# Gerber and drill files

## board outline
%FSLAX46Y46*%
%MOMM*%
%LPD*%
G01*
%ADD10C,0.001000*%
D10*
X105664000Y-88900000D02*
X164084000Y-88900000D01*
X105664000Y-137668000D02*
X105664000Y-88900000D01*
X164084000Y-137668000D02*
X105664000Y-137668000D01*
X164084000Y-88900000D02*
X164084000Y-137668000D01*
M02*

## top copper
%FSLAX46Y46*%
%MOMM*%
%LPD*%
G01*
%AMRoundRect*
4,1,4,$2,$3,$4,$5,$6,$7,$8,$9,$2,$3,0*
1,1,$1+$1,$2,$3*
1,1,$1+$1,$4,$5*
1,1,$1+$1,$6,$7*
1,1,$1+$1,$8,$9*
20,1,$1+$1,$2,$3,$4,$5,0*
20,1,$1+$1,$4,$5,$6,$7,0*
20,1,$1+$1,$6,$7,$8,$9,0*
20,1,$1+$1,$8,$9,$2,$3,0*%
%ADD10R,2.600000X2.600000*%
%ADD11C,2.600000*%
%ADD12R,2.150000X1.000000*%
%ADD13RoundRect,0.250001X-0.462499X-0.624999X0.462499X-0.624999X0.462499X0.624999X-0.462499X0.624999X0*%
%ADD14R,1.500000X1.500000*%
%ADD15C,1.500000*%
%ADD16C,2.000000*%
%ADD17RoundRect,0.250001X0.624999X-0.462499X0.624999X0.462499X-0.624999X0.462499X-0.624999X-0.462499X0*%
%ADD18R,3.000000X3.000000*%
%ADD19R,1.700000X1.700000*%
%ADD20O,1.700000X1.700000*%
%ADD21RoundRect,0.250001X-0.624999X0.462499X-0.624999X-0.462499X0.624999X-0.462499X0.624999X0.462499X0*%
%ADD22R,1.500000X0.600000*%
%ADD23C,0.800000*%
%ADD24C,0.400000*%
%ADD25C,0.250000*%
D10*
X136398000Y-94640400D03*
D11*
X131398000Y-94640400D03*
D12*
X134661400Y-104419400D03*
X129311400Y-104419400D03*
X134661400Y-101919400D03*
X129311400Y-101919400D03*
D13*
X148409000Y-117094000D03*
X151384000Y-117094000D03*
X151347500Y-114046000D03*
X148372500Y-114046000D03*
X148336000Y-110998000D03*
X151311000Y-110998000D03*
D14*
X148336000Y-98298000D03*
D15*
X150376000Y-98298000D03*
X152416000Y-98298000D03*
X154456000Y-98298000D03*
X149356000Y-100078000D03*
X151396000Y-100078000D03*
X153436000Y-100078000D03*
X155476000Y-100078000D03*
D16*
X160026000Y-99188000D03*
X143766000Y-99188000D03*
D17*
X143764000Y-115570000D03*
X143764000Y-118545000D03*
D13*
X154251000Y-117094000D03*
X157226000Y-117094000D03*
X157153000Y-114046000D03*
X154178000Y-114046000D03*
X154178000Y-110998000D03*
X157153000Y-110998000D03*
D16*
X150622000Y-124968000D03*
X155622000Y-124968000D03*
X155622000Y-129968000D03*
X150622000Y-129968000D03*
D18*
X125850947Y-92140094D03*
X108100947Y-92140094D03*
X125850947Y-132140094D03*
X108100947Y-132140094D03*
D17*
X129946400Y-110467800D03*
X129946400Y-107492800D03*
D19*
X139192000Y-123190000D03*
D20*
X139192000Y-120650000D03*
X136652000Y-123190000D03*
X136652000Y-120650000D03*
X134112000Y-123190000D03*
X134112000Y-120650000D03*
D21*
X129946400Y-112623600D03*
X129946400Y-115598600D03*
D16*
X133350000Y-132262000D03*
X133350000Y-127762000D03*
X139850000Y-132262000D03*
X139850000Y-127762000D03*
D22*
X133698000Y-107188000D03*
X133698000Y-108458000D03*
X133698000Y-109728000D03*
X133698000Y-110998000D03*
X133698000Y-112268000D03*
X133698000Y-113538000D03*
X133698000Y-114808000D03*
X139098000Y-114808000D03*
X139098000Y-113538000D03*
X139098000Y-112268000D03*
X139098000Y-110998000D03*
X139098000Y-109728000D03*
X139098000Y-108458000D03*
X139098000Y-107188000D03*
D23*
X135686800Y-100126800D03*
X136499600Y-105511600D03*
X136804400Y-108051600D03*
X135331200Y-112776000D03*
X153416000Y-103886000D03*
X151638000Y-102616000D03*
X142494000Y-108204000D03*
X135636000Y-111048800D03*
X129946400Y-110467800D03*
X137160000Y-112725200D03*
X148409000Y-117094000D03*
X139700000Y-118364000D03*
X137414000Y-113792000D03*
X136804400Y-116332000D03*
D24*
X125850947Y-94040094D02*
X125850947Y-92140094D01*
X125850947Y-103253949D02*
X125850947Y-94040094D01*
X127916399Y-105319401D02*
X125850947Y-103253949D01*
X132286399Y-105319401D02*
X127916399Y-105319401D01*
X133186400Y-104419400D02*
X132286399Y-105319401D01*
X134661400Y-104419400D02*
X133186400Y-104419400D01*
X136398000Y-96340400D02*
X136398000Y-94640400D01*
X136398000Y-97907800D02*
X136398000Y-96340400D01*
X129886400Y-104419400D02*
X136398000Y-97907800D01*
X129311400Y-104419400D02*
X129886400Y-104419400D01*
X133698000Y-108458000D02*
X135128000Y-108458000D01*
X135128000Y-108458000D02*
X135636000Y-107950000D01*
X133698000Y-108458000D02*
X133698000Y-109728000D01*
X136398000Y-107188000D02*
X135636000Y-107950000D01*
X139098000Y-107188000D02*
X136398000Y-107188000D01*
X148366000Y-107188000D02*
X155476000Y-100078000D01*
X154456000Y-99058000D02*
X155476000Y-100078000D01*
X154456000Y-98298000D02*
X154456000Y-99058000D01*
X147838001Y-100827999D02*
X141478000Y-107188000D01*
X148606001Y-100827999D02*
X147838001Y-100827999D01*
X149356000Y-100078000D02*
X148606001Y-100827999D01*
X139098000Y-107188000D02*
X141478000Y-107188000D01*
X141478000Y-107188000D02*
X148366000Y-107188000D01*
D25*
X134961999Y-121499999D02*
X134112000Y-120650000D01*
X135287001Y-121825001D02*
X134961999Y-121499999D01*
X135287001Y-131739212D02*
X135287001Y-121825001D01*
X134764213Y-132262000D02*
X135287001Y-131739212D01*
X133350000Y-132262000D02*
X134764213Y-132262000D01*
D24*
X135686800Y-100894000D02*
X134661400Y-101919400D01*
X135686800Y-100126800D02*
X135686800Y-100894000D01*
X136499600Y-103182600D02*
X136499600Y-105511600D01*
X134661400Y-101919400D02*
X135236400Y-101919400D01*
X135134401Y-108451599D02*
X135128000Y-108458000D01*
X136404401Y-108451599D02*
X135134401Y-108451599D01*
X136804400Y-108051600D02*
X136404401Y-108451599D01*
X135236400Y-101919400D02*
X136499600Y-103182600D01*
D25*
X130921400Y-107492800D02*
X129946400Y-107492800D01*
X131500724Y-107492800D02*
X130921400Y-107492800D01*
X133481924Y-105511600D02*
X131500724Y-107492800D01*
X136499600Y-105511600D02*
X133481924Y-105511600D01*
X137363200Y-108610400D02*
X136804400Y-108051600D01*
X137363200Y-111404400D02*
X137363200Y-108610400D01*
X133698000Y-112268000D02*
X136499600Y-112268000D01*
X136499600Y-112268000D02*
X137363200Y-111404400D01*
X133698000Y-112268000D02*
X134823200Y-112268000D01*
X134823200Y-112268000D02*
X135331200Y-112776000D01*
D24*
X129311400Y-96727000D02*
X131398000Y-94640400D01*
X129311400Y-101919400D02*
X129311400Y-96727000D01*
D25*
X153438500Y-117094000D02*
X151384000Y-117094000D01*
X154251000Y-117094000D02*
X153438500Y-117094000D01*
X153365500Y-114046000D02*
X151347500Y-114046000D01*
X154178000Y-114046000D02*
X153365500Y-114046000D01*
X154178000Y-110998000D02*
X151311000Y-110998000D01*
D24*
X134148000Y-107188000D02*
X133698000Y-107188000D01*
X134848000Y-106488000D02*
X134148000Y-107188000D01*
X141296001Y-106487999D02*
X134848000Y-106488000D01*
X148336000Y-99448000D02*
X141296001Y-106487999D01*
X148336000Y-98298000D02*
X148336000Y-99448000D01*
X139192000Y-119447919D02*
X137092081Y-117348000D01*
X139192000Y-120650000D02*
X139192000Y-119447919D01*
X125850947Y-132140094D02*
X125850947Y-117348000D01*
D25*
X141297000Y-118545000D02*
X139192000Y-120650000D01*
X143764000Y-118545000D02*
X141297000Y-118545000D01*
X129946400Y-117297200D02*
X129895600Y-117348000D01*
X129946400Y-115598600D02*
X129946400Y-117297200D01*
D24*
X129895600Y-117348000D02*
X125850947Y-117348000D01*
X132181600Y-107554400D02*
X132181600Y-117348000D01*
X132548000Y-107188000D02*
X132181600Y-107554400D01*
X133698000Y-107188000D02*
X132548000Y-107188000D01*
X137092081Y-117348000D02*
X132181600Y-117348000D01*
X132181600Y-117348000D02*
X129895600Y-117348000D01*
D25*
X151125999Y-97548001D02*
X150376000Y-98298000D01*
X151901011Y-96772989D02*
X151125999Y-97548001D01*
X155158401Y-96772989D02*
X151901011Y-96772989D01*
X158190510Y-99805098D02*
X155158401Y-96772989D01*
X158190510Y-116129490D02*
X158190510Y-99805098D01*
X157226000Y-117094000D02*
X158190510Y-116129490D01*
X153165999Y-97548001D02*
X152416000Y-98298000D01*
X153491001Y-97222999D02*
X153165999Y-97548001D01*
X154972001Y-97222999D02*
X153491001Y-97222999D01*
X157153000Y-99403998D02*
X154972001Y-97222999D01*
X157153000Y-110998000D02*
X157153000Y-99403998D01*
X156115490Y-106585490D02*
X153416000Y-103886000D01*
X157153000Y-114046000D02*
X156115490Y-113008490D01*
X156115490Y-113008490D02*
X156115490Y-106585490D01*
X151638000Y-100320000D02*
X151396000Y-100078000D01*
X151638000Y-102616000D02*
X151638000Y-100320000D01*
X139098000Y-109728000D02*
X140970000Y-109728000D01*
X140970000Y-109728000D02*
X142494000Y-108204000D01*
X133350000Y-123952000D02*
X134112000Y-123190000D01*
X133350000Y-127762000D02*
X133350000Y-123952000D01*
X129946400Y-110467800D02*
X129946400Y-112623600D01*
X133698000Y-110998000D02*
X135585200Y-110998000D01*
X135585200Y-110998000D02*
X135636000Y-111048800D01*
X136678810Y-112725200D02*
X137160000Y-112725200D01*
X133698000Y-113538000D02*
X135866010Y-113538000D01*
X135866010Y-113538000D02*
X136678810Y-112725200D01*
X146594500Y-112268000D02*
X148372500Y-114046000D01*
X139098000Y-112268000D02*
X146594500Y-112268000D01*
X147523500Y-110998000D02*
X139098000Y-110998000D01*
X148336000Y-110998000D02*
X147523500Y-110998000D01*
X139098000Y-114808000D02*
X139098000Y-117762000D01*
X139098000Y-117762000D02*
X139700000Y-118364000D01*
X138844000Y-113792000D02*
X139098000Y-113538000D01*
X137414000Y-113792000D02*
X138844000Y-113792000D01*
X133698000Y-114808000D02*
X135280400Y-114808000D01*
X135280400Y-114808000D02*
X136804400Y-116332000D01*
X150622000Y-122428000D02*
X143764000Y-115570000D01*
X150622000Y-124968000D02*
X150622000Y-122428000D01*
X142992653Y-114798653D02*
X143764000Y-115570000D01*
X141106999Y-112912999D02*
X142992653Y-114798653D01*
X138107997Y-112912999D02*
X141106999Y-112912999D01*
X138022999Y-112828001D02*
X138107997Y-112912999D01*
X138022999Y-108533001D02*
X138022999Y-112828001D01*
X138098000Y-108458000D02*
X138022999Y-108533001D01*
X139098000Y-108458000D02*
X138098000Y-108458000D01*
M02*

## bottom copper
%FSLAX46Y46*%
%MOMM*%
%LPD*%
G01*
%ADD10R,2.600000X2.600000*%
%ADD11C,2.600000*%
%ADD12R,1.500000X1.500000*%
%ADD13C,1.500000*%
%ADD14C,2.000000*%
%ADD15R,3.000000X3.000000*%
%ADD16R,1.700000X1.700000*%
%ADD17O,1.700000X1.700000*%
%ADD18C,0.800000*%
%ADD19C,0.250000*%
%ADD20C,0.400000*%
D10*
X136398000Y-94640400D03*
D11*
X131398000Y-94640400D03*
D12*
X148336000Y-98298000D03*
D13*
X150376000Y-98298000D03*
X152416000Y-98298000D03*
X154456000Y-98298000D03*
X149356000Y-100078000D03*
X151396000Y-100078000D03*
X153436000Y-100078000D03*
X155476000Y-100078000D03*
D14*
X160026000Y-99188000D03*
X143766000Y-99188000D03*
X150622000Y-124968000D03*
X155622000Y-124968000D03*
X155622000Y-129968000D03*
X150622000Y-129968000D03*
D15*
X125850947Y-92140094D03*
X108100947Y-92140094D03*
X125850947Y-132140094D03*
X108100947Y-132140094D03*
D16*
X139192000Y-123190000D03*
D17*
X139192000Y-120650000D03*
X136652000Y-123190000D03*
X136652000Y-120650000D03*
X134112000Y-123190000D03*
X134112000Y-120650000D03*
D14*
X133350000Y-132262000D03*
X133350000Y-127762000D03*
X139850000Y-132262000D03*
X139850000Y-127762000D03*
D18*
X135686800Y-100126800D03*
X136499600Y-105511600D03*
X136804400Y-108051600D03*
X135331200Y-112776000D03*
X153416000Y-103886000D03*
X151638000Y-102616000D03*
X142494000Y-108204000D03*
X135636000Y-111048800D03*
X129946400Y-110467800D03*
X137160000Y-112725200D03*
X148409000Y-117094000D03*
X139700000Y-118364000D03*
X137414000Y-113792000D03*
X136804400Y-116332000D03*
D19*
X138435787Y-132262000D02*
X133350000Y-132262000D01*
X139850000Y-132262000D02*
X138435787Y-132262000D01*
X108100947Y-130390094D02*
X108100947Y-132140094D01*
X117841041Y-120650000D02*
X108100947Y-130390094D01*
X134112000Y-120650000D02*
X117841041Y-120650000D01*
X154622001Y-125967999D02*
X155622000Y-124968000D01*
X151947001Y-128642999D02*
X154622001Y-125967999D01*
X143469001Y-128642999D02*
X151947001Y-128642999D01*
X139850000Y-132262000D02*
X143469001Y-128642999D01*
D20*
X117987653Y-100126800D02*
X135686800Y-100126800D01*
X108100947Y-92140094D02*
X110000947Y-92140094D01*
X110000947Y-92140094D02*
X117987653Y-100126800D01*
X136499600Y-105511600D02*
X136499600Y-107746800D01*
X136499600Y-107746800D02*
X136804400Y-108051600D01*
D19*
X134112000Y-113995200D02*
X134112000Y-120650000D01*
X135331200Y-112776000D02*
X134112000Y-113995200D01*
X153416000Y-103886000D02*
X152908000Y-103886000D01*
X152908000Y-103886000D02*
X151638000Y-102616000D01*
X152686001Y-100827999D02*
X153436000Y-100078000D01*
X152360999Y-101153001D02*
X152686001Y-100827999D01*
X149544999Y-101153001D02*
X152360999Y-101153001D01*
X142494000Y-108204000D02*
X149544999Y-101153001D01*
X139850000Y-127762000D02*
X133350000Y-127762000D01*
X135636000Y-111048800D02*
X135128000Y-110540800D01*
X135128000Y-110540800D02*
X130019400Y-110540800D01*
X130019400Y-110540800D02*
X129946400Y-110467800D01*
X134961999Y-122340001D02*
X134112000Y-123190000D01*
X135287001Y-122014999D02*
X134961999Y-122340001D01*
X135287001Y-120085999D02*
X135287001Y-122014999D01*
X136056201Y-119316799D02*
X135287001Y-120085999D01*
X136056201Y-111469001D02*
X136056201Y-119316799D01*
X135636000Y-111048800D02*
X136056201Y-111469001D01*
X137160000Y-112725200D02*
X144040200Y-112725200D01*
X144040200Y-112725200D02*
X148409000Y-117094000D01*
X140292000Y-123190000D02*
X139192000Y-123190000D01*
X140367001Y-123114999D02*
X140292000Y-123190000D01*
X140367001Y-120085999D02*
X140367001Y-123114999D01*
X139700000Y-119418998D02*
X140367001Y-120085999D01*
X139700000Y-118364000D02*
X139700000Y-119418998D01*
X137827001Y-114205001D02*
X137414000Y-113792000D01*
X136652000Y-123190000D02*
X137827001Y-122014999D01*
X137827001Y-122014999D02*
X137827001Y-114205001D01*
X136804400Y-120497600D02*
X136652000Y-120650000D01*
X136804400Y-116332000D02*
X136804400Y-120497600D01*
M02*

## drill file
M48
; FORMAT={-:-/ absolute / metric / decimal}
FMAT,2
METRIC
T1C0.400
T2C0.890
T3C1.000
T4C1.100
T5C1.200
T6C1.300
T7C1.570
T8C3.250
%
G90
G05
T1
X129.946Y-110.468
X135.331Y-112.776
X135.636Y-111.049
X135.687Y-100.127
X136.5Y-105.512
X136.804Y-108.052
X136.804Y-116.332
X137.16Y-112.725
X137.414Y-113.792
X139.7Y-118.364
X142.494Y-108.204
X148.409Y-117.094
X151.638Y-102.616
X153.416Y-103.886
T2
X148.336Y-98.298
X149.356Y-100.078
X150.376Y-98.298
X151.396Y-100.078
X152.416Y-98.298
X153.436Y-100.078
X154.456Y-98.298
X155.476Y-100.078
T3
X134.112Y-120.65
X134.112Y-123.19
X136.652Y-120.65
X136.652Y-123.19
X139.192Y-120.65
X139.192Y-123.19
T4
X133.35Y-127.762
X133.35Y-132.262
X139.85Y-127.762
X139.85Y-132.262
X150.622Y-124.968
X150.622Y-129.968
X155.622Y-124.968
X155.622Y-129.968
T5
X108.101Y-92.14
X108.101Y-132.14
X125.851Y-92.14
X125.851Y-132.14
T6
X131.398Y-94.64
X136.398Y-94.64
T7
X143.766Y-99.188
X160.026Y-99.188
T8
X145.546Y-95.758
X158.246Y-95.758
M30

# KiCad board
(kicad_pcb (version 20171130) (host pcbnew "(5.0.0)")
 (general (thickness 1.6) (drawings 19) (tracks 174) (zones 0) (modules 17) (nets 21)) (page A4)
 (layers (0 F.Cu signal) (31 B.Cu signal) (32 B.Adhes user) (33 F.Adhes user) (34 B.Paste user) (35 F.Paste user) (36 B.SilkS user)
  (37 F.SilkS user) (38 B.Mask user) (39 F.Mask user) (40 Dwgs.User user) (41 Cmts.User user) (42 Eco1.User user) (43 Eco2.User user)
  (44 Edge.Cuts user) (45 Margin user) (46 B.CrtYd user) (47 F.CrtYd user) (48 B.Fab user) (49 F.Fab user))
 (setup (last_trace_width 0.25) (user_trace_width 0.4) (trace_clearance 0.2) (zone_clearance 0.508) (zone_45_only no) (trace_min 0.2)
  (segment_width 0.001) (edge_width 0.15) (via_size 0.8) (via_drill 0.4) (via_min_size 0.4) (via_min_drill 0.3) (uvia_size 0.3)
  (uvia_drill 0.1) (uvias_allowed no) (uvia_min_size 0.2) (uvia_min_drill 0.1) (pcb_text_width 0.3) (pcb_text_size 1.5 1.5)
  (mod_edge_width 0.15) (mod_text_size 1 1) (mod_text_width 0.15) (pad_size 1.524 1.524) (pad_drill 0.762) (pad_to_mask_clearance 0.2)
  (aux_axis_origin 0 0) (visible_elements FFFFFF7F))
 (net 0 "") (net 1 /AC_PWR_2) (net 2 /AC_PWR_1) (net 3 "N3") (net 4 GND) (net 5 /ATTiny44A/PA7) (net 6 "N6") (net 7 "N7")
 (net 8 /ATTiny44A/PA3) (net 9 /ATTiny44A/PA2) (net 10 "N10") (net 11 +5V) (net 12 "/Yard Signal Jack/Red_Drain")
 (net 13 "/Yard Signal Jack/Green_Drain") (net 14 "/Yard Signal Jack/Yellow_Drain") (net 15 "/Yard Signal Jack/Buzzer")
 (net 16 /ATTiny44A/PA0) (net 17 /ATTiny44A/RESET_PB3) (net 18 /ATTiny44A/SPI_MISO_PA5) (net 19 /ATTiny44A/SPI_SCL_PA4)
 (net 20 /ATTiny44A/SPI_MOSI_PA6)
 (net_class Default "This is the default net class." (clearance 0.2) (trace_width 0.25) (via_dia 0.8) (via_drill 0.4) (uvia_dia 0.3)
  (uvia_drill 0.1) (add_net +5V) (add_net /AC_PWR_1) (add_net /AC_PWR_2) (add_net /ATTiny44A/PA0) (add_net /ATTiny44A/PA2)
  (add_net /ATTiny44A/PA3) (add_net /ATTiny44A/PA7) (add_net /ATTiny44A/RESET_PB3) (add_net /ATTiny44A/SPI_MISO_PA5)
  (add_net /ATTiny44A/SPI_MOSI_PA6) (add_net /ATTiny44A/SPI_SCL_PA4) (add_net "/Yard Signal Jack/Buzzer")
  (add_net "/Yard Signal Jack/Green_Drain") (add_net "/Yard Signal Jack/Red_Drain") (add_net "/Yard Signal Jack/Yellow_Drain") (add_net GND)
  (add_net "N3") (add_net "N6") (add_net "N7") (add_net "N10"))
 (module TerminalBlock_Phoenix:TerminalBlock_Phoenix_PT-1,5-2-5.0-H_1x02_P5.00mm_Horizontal (layer F.Cu) (at 136.398 94.6404 180)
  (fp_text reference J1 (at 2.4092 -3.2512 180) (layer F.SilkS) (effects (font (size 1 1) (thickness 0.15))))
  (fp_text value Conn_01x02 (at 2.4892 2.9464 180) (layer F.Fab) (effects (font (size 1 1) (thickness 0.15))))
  (pad 1 thru_hole rect (at 0 0 180) (size 2.6 2.6) (drill 1.3) (layers *.Cu *.Mask) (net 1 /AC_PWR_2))
  (pad 2 thru_hole circle (at 5 0 180) (size 2.6 2.6) (drill 1.3) (layers *.Cu *.Mask) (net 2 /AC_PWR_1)))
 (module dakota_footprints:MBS (layer F.Cu) (at 132.0292 103.124)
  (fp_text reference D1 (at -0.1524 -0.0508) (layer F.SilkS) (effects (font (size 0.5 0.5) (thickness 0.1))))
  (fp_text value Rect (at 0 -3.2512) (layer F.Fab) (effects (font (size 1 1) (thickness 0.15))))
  (pad 1 smd rect (at 2.6322 1.2954 90) (size 1 2.15) (layers F.Cu F.Paste F.Mask) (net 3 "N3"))
  (pad 3 smd rect (at -2.7178 1.2954 90) (size 1 2.15) (layers F.Cu F.Paste F.Mask) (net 1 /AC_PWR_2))
  (pad 2 smd rect (at 2.6322 -1.2046 90) (size 1 2.15) (layers F.Cu F.Paste F.Mask) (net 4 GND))
  (pad 4 smd rect (at -2.7178 -1.2046 90) (size 1 2.15) (layers F.Cu F.Paste F.Mask) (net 2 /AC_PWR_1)))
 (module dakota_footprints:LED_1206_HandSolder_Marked (layer F.Cu) (at 149.8965 117.094)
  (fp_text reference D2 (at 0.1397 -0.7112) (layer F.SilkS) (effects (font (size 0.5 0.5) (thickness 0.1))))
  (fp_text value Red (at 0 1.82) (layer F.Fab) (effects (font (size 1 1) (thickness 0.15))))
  (pad 1 smd roundrect (at -1.4875 0) (size 1.425 1.75) (layers F.Cu F.Paste F.Mask) (roundrect_rratio 0.175439) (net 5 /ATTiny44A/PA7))
  (pad 2 smd roundrect (at 1.4875 0) (size 1.425 1.75) (layers F.Cu F.Paste F.Mask) (roundrect_rratio 0.175439) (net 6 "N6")))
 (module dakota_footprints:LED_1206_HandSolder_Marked (layer F.Cu) (at 149.86 114.046)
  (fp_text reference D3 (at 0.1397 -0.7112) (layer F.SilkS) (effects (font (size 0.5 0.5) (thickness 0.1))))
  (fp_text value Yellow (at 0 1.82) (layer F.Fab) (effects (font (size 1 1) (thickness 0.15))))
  (pad 2 smd roundrect (at 1.4875 0) (size 1.425 1.75) (layers F.Cu F.Paste F.Mask) (roundrect_rratio 0.175439) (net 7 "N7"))
  (pad 1 smd roundrect (at -1.4875 0) (size 1.425 1.75) (layers F.Cu F.Paste F.Mask) (roundrect_rratio 0.175439) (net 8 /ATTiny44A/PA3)))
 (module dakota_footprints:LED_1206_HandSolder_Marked (layer F.Cu) (at 149.8235 110.998)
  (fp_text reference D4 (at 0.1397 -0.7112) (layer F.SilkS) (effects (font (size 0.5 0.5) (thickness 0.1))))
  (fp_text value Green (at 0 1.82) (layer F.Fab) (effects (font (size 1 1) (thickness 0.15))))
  (pad 1 smd roundrect (at -1.4875 0) (size 1.425 1.75) (layers F.Cu F.Paste F.Mask) (roundrect_rratio 0.175439) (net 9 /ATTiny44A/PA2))
  (pad 2 smd roundrect (at 1.4875 0) (size 1.425 1.75) (layers F.Cu F.Paste F.Mask) (roundrect_rratio 0.175439) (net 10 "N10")))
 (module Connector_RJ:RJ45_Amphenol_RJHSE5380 (layer F.Cu) (at 148.336 98.298)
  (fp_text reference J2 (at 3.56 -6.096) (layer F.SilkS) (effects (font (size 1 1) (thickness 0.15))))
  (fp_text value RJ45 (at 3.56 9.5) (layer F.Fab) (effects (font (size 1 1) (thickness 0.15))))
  (pad 1 thru_hole rect (at 0 0) (size 1.5 1.5) (drill 0.89) (layers *.Cu *.Mask) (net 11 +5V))
  (pad 3 thru_hole circle (at 2.04 0) (size 1.5 1.5) (drill 0.89) (layers *.Cu *.Mask) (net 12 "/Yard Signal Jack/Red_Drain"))
  (pad 5 thru_hole circle (at 4.08 0) (size 1.5 1.5) (drill 0.89) (layers *.Cu *.Mask) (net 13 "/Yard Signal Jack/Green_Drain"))
  (pad 7 thru_hole circle (at 6.12 0) (size 1.5 1.5) (drill 0.89) (layers *.Cu *.Mask) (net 4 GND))
  (pad 2 thru_hole circle (at 1.02 1.78) (size 1.5 1.5) (drill 0.89) (layers *.Cu *.Mask) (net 4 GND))
  (pad 4 thru_hole circle (at 3.06 1.78) (size 1.5 1.5) (drill 0.89) (layers *.Cu *.Mask) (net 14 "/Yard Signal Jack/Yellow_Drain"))
  (pad 6 thru_hole circle (at 5.1 1.78) (size 1.5 1.5) (drill 0.89) (layers *.Cu *.Mask) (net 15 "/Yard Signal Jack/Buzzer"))
  (pad 8 thru_hole circle (at 7.14 1.78) (size 1.5 1.5) (drill 0.89) (layers *.Cu *.Mask) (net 4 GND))
  (pad "" np_thru_hole circle (at -2.79 -2.54) (size 3.25 3.25) (drill 3.25) (layers *.Cu *.Mask))
  (pad "" np_thru_hole circle (at 9.91 -2.54) (size 3.25 3.25) (drill 3.25) (layers *.Cu *.Mask))
  (pad SH thru_hole circle (at 11.69 0.89) (size 2 2) (drill 1.57) (layers *.Cu *.Mask))
  (pad SH thru_hole circle (at -4.57 0.89) (size 2 2) (drill 1.57) (layers *.Cu *.Mask)))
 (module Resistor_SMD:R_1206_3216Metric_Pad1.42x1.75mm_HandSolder (layer F.Cu) (at 143.764 117.0575 90)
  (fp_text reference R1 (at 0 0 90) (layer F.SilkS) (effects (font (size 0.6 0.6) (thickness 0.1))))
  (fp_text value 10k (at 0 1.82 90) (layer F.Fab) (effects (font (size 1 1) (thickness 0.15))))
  (pad 2 smd roundrect (at 1.4875 0 90) (size 1.425 1.75) (layers F.Cu F.Paste F.Mask) (roundrect_rratio 0.175439) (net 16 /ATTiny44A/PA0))
  (pad 1 smd roundrect (at -1.4875 0 90) (size 1.425 1.75) (layers F.Cu F.Paste F.Mask) (roundrect_rratio 0.175439) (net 11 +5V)))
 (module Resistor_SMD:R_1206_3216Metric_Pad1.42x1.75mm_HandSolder (layer F.Cu) (at 155.7385 117.094)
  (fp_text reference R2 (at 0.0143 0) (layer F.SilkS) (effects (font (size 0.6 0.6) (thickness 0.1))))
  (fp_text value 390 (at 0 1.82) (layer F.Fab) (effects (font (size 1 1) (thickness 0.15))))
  (pad 1 smd roundrect (at -1.4875 0) (size 1.425 1.75) (layers F.Cu F.Paste F.Mask) (roundrect_rratio 0.175439) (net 6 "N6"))
  (pad 2 smd roundrect (at 1.4875 0) (size 1.425 1.75) (layers F.Cu F.Paste F.Mask) (roundrect_rratio 0.175439)
   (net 12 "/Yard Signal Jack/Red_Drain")))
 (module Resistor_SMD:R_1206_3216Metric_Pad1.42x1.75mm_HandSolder (layer F.Cu) (at 155.6655 114.046)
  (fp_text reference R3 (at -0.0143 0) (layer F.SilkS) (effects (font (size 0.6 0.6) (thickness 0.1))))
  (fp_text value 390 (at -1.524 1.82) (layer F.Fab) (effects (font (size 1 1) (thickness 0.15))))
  (pad 2 smd roundrect (at 1.4875 0) (size 1.425 1.75) (layers F.Cu F.Paste F.Mask) (roundrect_rratio 0.175439)
   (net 14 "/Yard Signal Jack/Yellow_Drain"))
  (pad 1 smd roundrect (at -1.4875 0) (size 1.425 1.75) (layers F.Cu F.Paste F.Mask) (roundrect_rratio 0.175439) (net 7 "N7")))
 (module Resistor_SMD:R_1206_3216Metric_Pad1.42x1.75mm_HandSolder (layer F.Cu) (at 155.6655 110.998)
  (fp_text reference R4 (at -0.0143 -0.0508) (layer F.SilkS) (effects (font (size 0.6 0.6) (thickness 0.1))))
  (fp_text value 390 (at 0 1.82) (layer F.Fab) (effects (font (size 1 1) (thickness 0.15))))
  (pad 1 smd roundrect (at -1.4875 0) (size 1.425 1.75) (layers F.Cu F.Paste F.Mask) (roundrect_rratio 0.175439) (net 10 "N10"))
  (pad 2 smd roundrect (at 1.4875 0) (size 1.425 1.75) (layers F.Cu F.Paste F.Mask) (roundrect_rratio 0.175439)
   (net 13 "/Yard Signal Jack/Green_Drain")))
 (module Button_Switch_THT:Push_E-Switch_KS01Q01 (layer F.Cu) (at 150.622 124.968)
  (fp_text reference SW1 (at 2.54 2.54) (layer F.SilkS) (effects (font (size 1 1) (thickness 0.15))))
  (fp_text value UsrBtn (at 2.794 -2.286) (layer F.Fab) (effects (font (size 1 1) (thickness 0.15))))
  (pad 1 thru_hole circle (at 0 0) (size 2 2) (drill 1.1) (layers *.Cu *.Mask) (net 16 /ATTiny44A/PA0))
  (pad 2 thru_hole circle (at 5 0) (size 2 2) (drill 1.1) (layers *.Cu *.Mask) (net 4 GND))
  (pad 4 thru_hole circle (at 5 5) (size 2 2) (drill 1.1) (layers *.Cu *.Mask))
  (pad 3 thru_hole circle (at 0 5) (size 2 2) (drill 1.1) (layers *.Cu *.Mask)))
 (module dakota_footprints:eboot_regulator (layer F.Cu) (at 125.850947 92.140094 270)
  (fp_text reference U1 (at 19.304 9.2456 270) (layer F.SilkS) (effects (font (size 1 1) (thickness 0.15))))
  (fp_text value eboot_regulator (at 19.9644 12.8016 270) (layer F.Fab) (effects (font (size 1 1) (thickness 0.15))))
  (pad 1 thru_hole rect (at 0 0 270) (size 3 3) (drill 1.2) (layers *.Cu *.Mask) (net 3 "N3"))
  (pad 2 thru_hole rect (at 0 17.75 270) (size 3 3) (drill 1.2) (layers *.Cu *.Mask) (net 4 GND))
  (pad 3 thru_hole rect (at 40 0 270) (size 3 3) (drill 1.2) (layers *.Cu *.Mask) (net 11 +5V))
  (pad 4 thru_hole rect (at 40 17.75 270) (size 3 3) (drill 1.2) (layers *.Cu *.Mask) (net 4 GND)))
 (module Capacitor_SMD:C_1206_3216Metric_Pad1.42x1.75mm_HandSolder (layer F.Cu) (at 129.9464 108.9803 90)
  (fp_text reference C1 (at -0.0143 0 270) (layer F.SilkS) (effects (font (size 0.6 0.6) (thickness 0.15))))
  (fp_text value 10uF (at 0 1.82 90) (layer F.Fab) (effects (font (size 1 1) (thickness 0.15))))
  (pad 1 smd roundrect (at -1.4875 0 90) (size 1.425 1.75) (layers F.Cu F.Paste F.Mask) (roundrect_rratio 0.175439)
   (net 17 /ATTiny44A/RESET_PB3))
  (pad 2 smd roundrect (at 1.4875 0 90) (size 1.425 1.75) (layers F.Cu F.Paste F.Mask) (roundrect_rratio 0.175439) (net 4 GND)))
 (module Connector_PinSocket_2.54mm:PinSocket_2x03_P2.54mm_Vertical (layer F.Cu) (at 139.192 123.19 270)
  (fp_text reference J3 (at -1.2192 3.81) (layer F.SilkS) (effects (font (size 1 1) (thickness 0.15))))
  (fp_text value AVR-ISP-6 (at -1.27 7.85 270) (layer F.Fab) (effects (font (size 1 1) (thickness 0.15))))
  (pad 1 thru_hole rect (at 0 0 270) (size 1.7 1.7) (drill 1) (layers *.Cu *.Mask) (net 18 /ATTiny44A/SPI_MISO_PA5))
  (pad 2 thru_hole oval (at -2.54 0 270) (size 1.7 1.7) (drill 1) (layers *.Cu *.Mask) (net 11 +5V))
  (pad 3 thru_hole oval (at 0 2.54 270) (size 1.7 1.7) (drill 1) (layers *.Cu *.Mask) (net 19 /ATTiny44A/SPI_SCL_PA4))
  (pad 4 thru_hole oval (at -2.54 2.54 270) (size 1.7 1.7) (drill 1) (layers *.Cu *.Mask) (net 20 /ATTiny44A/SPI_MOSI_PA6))
  (pad 5 thru_hole oval (at 0 5.08 270) (size 1.7 1.7) (drill 1) (layers *.Cu *.Mask) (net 17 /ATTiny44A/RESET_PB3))
  (pad 6 thru_hole oval (at -2.54 5.08 270) (size 1.7 1.7) (drill 1) (layers *.Cu *.Mask) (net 4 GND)))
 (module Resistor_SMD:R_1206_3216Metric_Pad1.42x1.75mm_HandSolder (layer F.Cu) (at 129.9464 114.1111 270)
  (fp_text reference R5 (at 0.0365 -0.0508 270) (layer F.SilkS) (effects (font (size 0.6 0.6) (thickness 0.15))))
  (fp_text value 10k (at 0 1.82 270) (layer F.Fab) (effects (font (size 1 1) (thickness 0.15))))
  (pad 1 smd roundrect (at -1.4875 0 270) (size 1.425 1.75) (layers F.Cu F.Paste F.Mask) (roundrect_rratio 0.175439)
   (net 17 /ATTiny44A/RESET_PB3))
  (pad 2 smd roundrect (at 1.4875 0 270) (size 1.425 1.75) (layers F.Cu F.Paste F.Mask) (roundrect_rratio 0.175439) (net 11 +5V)))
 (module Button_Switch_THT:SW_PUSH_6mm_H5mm (layer F.Cu) (at 133.35 127.762)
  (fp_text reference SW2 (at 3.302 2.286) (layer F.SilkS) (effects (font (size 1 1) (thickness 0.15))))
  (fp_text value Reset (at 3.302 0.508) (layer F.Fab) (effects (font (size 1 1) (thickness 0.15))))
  (pad 2 thru_hole circle (at 0 4.5 90) (size 2 2) (drill 1.1) (layers *.Cu *.Mask) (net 4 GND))
  (pad 1 thru_hole circle (at 0 0 90) (size 2 2) (drill 1.1) (layers *.Cu *.Mask) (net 17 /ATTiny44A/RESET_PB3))
  (pad 2 thru_hole circle (at 6.5 4.5 90) (size 2 2) (drill 1.1) (layers *.Cu *.Mask) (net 4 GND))
  (pad 1 thru_hole circle (at 6.5 0 90) (size 2 2) (drill 1.1) (layers *.Cu *.Mask) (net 17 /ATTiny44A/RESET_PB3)))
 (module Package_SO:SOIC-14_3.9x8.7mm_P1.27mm (layer F.Cu) (at 136.398 110.998)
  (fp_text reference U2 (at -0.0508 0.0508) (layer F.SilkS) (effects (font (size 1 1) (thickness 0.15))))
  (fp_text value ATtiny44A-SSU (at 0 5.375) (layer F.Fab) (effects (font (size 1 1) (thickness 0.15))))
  (pad 1 smd rect (at -2.7 -3.81) (size 1.5 0.6) (layers F.Cu F.Paste F.Mask) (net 11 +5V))
  (pad 2 smd rect (at -2.7 -2.54) (size 1.5 0.6) (layers F.Cu F.Paste F.Mask) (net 4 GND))
  (pad 3 smd rect (at -2.7 -1.27) (size 1.5 0.6) (layers F.Cu F.Paste F.Mask) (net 4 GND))
  (pad 4 smd rect (at -2.7 0) (size 1.5 0.6) (layers F.Cu F.Paste F.Mask) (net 17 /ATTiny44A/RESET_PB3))
  (pad 5 smd rect (at -2.7 1.27) (size 1.5 0.6) (layers F.Cu F.Paste F.Mask) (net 4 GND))
  (pad 6 smd rect (at -2.7 2.54) (size 1.5 0.6) (layers F.Cu F.Paste F.Mask) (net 5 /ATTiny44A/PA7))
  (pad 7 smd rect (at -2.7 3.81) (size 1.5 0.6) (layers F.Cu F.Paste F.Mask) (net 20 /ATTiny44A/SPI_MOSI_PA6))
  (pad 8 smd rect (at 2.7 3.81) (size 1.5 0.6) (layers F.Cu F.Paste F.Mask) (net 18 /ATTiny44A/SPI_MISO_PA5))
  (pad 9 smd rect (at 2.7 2.54) (size 1.5 0.6) (layers F.Cu F.Paste F.Mask) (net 19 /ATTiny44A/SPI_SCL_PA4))
  (pad 10 smd rect (at 2.7 1.27) (size 1.5 0.6) (layers F.Cu F.Paste F.Mask) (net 8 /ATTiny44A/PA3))
  (pad 11 smd rect (at 2.7 0) (size 1.5 0.6) (layers F.Cu F.Paste F.Mask) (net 9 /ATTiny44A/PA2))
  (pad 12 smd rect (at 2.7 -1.27) (size 1.5 0.6) (layers F.Cu F.Paste F.Mask) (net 15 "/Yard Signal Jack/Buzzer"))
  (pad 13 smd rect (at 2.7 -2.54) (size 1.5 0.6) (layers F.Cu F.Paste F.Mask) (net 16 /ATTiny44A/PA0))
  (pad 14 smd rect (at 2.7 -3.81) (size 1.5 0.6) (layers F.Cu F.Paste F.Mask) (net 4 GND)))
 (gr_line (start 105.664 88.9) (end 164.084 88.9) (layer Edge.Cuts) (width 0.001))
 (gr_line (start 105.664 137.668) (end 105.664 88.9) (layer Edge.Cuts) (width 0.001))
 (gr_line (start 164.084 137.668) (end 105.664 137.668) (layer Edge.Cuts) (width 0.001))
 (gr_line (start 164.084 88.9) (end 164.084 137.668) (layer Edge.Cuts) (width 0.001))
 (segment (start 125.850947 94.040094) (end 125.850947 92.140094) (width 0.4) (layer F.Cu) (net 3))
 (segment (start 125.850947 103.253949) (end 125.850947 94.040094) (width 0.4) (layer F.Cu) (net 3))
 (segment (start 127.916399 105.319401) (end 125.850947 103.253949) (width 0.4) (layer F.Cu) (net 3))
 (segment (start 132.286399 105.319401) (end 127.916399 105.319401) (width 0.4) (layer F.Cu) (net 3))
 (segment (start 133.1864 104.4194) (end 132.286399 105.319401) (width 0.4) (layer F.Cu) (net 3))
 (segment (start 134.6614 104.4194) (end 133.1864 104.4194) (width 0.4) (layer F.Cu) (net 3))
 (segment (start 136.398 96.3404) (end 136.398 94.6404) (width 0.4) (layer F.Cu) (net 1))
 (segment (start 136.398 97.9078) (end 136.398 96.3404) (width 0.4) (layer F.Cu) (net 1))
 (segment (start 129.8864 104.4194) (end 136.398 97.9078) (width 0.4) (layer F.Cu) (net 1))
 (segment (start 129.3114 104.4194) (end 129.8864 104.4194) (width 0.4) (layer F.Cu) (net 1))
 (segment (start 133.698 108.458) (end 135.128 108.458) (width 0.4) (layer F.Cu) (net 4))
 (segment (start 135.128 108.458) (end 135.636 107.95) (width 0.4) (layer F.Cu) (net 4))
 (segment (start 133.698 108.458) (end 133.698 109.728) (width 0.4) (layer F.Cu) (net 4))
 (segment (start 136.398 107.188) (end 135.636 107.95) (width 0.4) (layer F.Cu) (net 4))
 (segment (start 139.098 107.188) (end 136.398 107.188) (width 0.4) (layer F.Cu) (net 4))
 (segment (start 148.366 107.188) (end 155.476 100.078) (width 0.4) (layer F.Cu) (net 4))
 (segment (start 154.456 99.058) (end 155.476 100.078) (width 0.4) (layer F.Cu) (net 4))
 (segment (start 154.456 98.298) (end 154.456 99.058) (width 0.4) (layer F.Cu) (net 4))
 (segment (start 147.838001 100.827999) (end 141.478 107.188) (width 0.4) (layer F.Cu) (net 4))
 (segment (start 148.606001 100.827999) (end 147.838001 100.827999) (width 0.4) (layer F.Cu) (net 4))
 (segment (start 149.356 100.078) (end 148.606001 100.827999) (width 0.4) (layer F.Cu) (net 4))
 (segment (start 139.098 107.188) (end 141.478 107.188) (width 0.4) (layer F.Cu) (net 4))
 (segment (start 141.478 107.188) (end 148.366 107.188) (width 0.4) (layer F.Cu) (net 4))
 (segment (start 134.961999 121.499999) (end 134.112 120.65) (width 0.25) (layer F.Cu) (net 4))
 (segment (start 135.287001 121.825001) (end 134.961999 121.499999) (width 0.25) (layer F.Cu) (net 4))
 (segment (start 135.287001 131.739212) (end 135.287001 121.825001) (width 0.25) (layer F.Cu) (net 4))
 (segment (start 134.764213 132.262) (end 135.287001 131.739212) (width 0.25) (layer F.Cu) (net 4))
 (segment (start 133.35 132.262) (end 134.764213 132.262) (width 0.25) (layer F.Cu) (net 4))
 (segment (start 138.435787 132.262) (end 133.35 132.262) (width 0.25) (layer B.Cu) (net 4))
 (segment (start 139.85 132.262) (end 138.435787 132.262) (width 0.25) (layer B.Cu) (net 4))
 (segment (start 108.100947 130.390094) (end 108.100947 132.140094) (width 0.25) (layer B.Cu) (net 4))
 (segment (start 117.841041 120.65) (end 108.100947 130.390094) (width 0.25) (layer B.Cu) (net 4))
 (segment (start 134.112 120.65) (end 117.841041 120.65) (width 0.25) (layer B.Cu) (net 4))
 (segment (start 154.622001 125.967999) (end 155.622 124.968) (width 0.25) (layer B.Cu) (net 4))
 (segment (start 151.947001 128.642999) (end 154.622001 125.967999) (width 0.25) (layer B.Cu) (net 4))
 (segment (start 143.469001 128.642999) (end 151.947001 128.642999) (width 0.25) (layer B.Cu) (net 4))
 (segment (start 139.85 132.262) (end 143.469001 128.642999) (width 0.25) (layer B.Cu) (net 4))
 (via (at 135.6868 100.1268) (size 0.8) (drill 0.4) (layers F.Cu B.Cu) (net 4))
 (segment (start 117.987653 100.1268) (end 135.6868 100.1268) (width 0.4) (layer B.Cu) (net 4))
 (segment (start 108.100947 92.140094) (end 110.000947 92.140094) (width 0.4) (layer B.Cu) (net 4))
 (segment (start 110.000947 92.140094) (end 117.987653 100.1268) (width 0.4) (layer B.Cu) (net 4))
 (segment (start 135.6868 100.894) (end 134.6614 101.9194) (width 0.4) (layer F.Cu) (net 4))
 (segment (start 135.6868 100.1268) (end 135.6868 100.894) (width 0.4) (layer F.Cu) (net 4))
 (via (at 136.4996 105.5116) (size 0.8) (drill 0.4) (layers F.Cu B.Cu) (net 4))
 (segment (start 136.4996 103.1826) (end 136.4996 105.5116) (width 0.4) (layer F.Cu) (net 4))
 (segment (start 134.6614 101.9194) (end 135.2364 101.9194) (width 0.4) (layer F.Cu) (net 4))
 (via (at 136.8044 108.0516) (size 0.8) (drill 0.4) (layers F.Cu B.Cu) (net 4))
 (segment (start 136.4996 105.5116) (end 136.4996 107.7468) (width 0.4) (layer B.Cu) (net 4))
 (segment (start 136.4996 107.7468) (end 136.8044 108.0516) (width 0.4) (layer B.Cu) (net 4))
 (segment (start 135.134401 108.451599) (end 135.128 108.458) (width 0.4) (layer F.Cu) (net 4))
 (segment (start 136.404401 108.451599) (end 135.134401 108.451599) (width 0.4) (layer F.Cu) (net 4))
 (segment (start 136.8044 108.0516) (end 136.404401 108.451599) (width 0.4) (layer F.Cu) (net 4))
 (segment (start 135.2364 101.9194) (end 136.4996 103.1826) (width 0.4) (layer F.Cu) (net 4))
 (segment (start 130.9214 107.4928) (end 129.9464 107.4928) (width 0.25) (layer F.Cu) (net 4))
 (segment (start 131.500724 107.4928) (end 130.9214 107.4928) (width 0.25) (layer F.Cu) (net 4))
 (segment (start 133.481924 105.5116) (end 131.500724 107.4928) (width 0.25) (layer F.Cu) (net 4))
 (segment (start 136.4996 105.5116) (end 133.481924 105.5116) (width 0.25) (layer F.Cu) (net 4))
 (segment (start 137.3632 108.6104) (end 136.8044 108.0516) (width 0.25) (layer F.Cu) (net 4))
 (segment (start 137.3632 111.4044) (end 137.3632 108.6104) (width 0.25) (layer F.Cu) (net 4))
 (segment (start 133.698 112.268) (end 136.4996 112.268) (width 0.25) (layer F.Cu) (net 4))
 (segment (start 136.4996 112.268) (end 137.3632 111.4044) (width 0.25) (layer F.Cu) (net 4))
 (via (at 135.3312 112.776) (size 0.8) (drill 0.4) (layers F.Cu B.Cu) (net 4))
 (segment (start 133.698 112.268) (end 134.8232 112.268) (width 0.25) (layer F.Cu) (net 4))
 (segment (start 134.8232 112.268) (end 135.3312 112.776) (width 0.25) (layer F.Cu) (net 4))
 (segment (start 134.112 113.9952) (end 134.112 120.65) (width 0.25) (layer B.Cu) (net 4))
 (segment (start 135.3312 112.776) (end 134.112 113.9952) (width 0.25) (layer B.Cu) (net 4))
 (segment (start 129.3114 96.727) (end 131.398 94.6404) (width 0.4) (layer F.Cu) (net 2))
 (segment (start 129.3114 101.9194) (end 129.3114 96.727) (width 0.4) (layer F.Cu) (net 2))
 (segment (start 153.4385 117.094) (end 151.384 117.094) (width 0.25) (layer F.Cu) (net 6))
 (segment (start 154.251 117.094) (end 153.4385 117.094) (width 0.25) (layer F.Cu) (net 6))
 (segment (start 153.3655 114.046) (end 151.3475 114.046) (width 0.25) (layer F.Cu) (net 7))
 (segment (start 154.178 114.046) (end 153.3655 114.046) (width 0.25) (layer F.Cu) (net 7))
 (segment (start 154.178 110.998) (end 151.311 110.998) (width 0.25) (layer F.Cu) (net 10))
 (segment (start 134.148 107.188) (end 133.698 107.188) (width 0.4) (layer F.Cu) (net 11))
 (segment (start 134.848 106.488) (end 134.148 107.188) (width 0.4) (layer F.Cu) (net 11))
 (segment (start 141.296001 106.487999) (end 134.848 106.488) (width 0.4) (layer F.Cu) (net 11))
 (segment (start 148.336 99.448) (end 141.296001 106.487999) (width 0.4) (layer F.Cu) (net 11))
 (segment (start 148.336 98.298) (end 148.336 99.448) (width 0.4) (layer F.Cu) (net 11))
 (segment (start 139.192 119.447919) (end 137.092081 117.348) (width 0.4) (layer F.Cu) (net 11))
 (segment (start 139.192 120.65) (end 139.192 119.447919) (width 0.4) (layer F.Cu) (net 11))
 (segment (start 125.850947 132.140094) (end 125.850947 117.348) (width 0.4) (layer F.Cu) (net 11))
 (segment (start 141.297 118.545) (end 139.192 120.65) (width 0.25) (layer F.Cu) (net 11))
 (segment (start 143.764 118.545) (end 141.297 118.545) (width 0.25) (layer F.Cu) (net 11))
 (segment (start 129.9464 117.2972) (end 129.8956 117.348) (width 0.25) (layer F.Cu) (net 11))
 (segment (start 129.9464 115.5986) (end 129.9464 117.2972) (width 0.25) (layer F.Cu) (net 11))
 (segment (start 129.8956 117.348) (end 125.850947 117.348) (width 0.4) (layer F.Cu) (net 11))
 (segment (start 132.1816 107.5544) (end 132.1816 117.348) (width 0.4) (layer F.Cu) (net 11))
 (segment (start 132.548 107.188) (end 132.1816 107.5544) (width 0.4) (layer F.Cu) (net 11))
 (segment (start 133.698 107.188) (end 132.548 107.188) (width 0.4) (layer F.Cu) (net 11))
 (segment (start 137.092081 117.348) (end 132.1816 117.348) (width 0.4) (layer F.Cu) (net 11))
 (segment (start 132.1816 117.348) (end 129.8956 117.348) (width 0.4) (layer F.Cu) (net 11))
 (segment (start 151.125999 97.548001) (end 150.376 98.298) (width 0.25) (layer F.Cu) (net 12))
 (segment (start 151.901011 96.772989) (end 151.125999 97.548001) (width 0.25) (layer F.Cu) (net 12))
 (segment (start 155.158401 96.772989) (end 151.901011 96.772989) (width 0.25) (layer F.Cu) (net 12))
 (segment (start 158.19051 99.805098) (end 155.158401 96.772989) (width 0.25) (layer F.Cu) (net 12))
 (segment (start 158.19051 116.12949) (end 158.19051 99.805098) (width 0.25) (layer F.Cu) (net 12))
 (segment (start 157.226 117.094) (end 158.19051 116.12949) (width 0.25) (layer F.Cu) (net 12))
 (segment (start 153.165999 97.548001) (end 152.416 98.298) (width 0.25) (layer F.Cu) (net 13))
 (segment (start 153.491001 97.222999) (end 153.165999 97.548001) (width 0.25) (layer F.Cu) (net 13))
 (segment (start 154.972001 97.222999) (end 153.491001 97.222999) (width 0.25) (layer F.Cu) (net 13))
 (segment (start 157.153 99.403998) (end 154.972001 97.222999) (width 0.25) (layer F.Cu) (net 13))
 (segment (start 157.153 110.998) (end 157.153 99.403998) (width 0.25) (layer F.Cu) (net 13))
 (via (at 153.416 103.886) (size 0.8) (drill 0.4) (layers F.Cu B.Cu) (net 14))
 (segment (start 156.11549 106.58549) (end 153.416 103.886) (width 0.25) (layer F.Cu) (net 14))
 (segment (start 157.153 114.046) (end 156.11549 113.00849) (width 0.25) (layer F.Cu) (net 14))
 (segment (start 156.11549 113.00849) (end 156.11549 106.58549) (width 0.25) (layer F.Cu) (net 14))
 (via (at 151.638 102.616) (size 0.8) (drill 0.4) (layers F.Cu B.Cu) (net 14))
 (segment (start 153.416 103.886) (end 152.908 103.886) (width 0.25) (layer B.Cu) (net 14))
 (segment (start 152.908 103.886) (end 151.638 102.616) (width 0.25) (layer B.Cu) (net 14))
 (segment (start 151.638 100.32) (end 151.396 100.078) (width 0.25) (layer F.Cu) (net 14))
 (segment (start 151.638 102.616) (end 151.638 100.32) (width 0.25) (layer F.Cu) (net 14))
 (via (at 142.494 108.204) (size 0.8) (drill 0.4) (layers F.Cu B.Cu) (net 15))
 (segment (start 139.098 109.728) (end 140.97 109.728) (width 0.25) (layer F.Cu) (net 15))
 (segment (start 140.97 109.728) (end 142.494 108.204) (width 0.25) (layer F.Cu) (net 15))
 (segment (start 152.686001 100.827999) (end 153.436 100.078) (width 0.25) (layer B.Cu) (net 15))
 (segment (start 152.360999 101.153001) (end 152.686001 100.827999) (width 0.25) (layer B.Cu) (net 15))
 (segment (start 149.544999 101.153001) (end 152.360999 101.153001) (width 0.25) (layer B.Cu) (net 15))
 (segment (start 142.494 108.204) (end 149.544999 101.153001) (width 0.25) (layer B.Cu) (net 15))
 (segment (start 133.35 123.952) (end 134.112 123.19) (width 0.25) (layer F.Cu) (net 17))
 (segment (start 133.35 127.762) (end 133.35 123.952) (width 0.25) (layer F.Cu) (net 17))
 (segment (start 139.85 127.762) (end 133.35 127.762) (width 0.25) (layer B.Cu) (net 17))
 (segment (start 129.9464 110.4678) (end 129.9464 112.6236) (width 0.25) (layer F.Cu) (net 17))
 (via (at 135.636 111.0488) (size 0.8) (drill 0.4) (layers F.Cu B.Cu) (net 17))
 (segment (start 133.698 110.998) (end 135.5852 110.998) (width 0.25) (layer F.Cu) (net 17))
 (segment (start 135.5852 110.998) (end 135.636 111.0488) (width 0.25) (layer F.Cu) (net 17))
 (segment (start 135.636 111.0488) (end 135.128 110.5408) (width 0.25) (layer B.Cu) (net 17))
 (via (at 129.9464 110.4678) (size 0.8) (drill 0.4) (layers F.Cu B.Cu) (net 17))
 (segment (start 135.128 110.5408) (end 130.0194 110.5408) (width 0.25) (layer B.Cu) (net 17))
 (segment (start 130.0194 110.5408) (end 129.9464 110.4678) (width 0.25) (layer B.Cu) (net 17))
 (segment (start 134.961999 122.340001) (end 134.112 123.19) (width 0.25) (layer B.Cu) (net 17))
 (segment (start 135.287001 122.014999) (end 134.961999 122.340001) (width 0.25) (layer B.Cu) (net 17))
 (segment (start 135.287001 120.085999) (end 135.287001 122.014999) (width 0.25) (layer B.Cu) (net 17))
 (segment (start 136.056201 119.316799) (end 135.287001 120.085999) (width 0.25) (layer B.Cu) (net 17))
 (segment (start 136.056201 111.469001) (end 136.056201 119.316799) (width 0.25) (layer B.Cu) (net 17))
 (segment (start 135.636 111.0488) (end 136.056201 111.469001) (width 0.25) (layer B.Cu) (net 17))
 (via (at 137.16 112.7252) (size 0.8) (drill 0.4) (layers F.Cu B.Cu) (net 5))
 (segment (start 136.67881 112.7252) (end 137.16 112.7252) (width 0.25) (layer F.Cu) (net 5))
 (segment (start 133.698 113.538) (end 135.86601 113.538) (width 0.25) (layer F.Cu) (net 5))
 (segment (start 135.86601 113.538) (end 136.67881 112.7252) (width 0.25) (layer F.Cu) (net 5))
 (via (at 148.409 117.094) (size 0.8) (drill 0.4) (layers F.Cu B.Cu) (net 5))
 (segment (start 137.16 112.7252) (end 144.0402 112.7252) (width 0.25) (layer B.Cu) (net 5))
 (segment (start 144.0402 112.7252) (end 148.409 117.094) (width 0.25) (layer B.Cu) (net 5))
 (segment (start 146.5945 112.268) (end 148.3725 114.046) (width 0.25) (layer F.Cu) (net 8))
 (segment (start 139.098 112.268) (end 146.5945 112.268) (width 0.25) (layer F.Cu) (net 8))
 (segment (start 147.5235 110.998) (end 139.098 110.998) (width 0.25) (layer F.Cu) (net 9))
 (segment (start 148.336 110.998) (end 147.5235 110.998) (width 0.25) (layer F.Cu) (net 9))
 (via (at 139.7 118.364) (size 0.8) (drill 0.4) (layers F.Cu B.Cu) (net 18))
 (segment (start 139.098 114.808) (end 139.098 117.762) (width 0.25) (layer F.Cu) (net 18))
 (segment (start 139.098 117.762) (end 139.7 118.364) (width 0.25) (layer F.Cu) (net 18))
 (segment (start 140.292 123.19) (end 139.192 123.19) (width 0.25) (layer B.Cu) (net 18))
 (segment (start 140.367001 123.114999) (end 140.292 123.19) (width 0.25) (layer B.Cu) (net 18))
 (segment (start 140.367001 120.085999) (end 140.367001 123.114999) (width 0.25) (layer B.Cu) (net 18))
 (segment (start 139.7 119.418998) (end 140.367001 120.085999) (width 0.25) (layer B.Cu) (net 18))
 (segment (start 139.7 118.364) (end 139.7 119.418998) (width 0.25) (layer B.Cu) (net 18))
 (via (at 137.414 113.792) (size 0.8) (drill 0.4) (layers F.Cu B.Cu) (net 19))
 (segment (start 137.827001 114.205001) (end 137.414 113.792) (width 0.25) (layer B.Cu) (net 19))
 (segment (start 136.652 123.19) (end 137.827001 122.014999) (width 0.25) (layer B.Cu) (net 19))
 (segment (start 137.827001 122.014999) (end 137.827001 114.205001) (width 0.25) (layer B.Cu) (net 19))
 (segment (start 138.844 113.792) (end 139.098 113.538) (width 0.25) (layer F.Cu) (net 19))
 (segment (start 137.414 113.792) (end 138.844 113.792) (width 0.25) (layer F.Cu) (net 19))
 (via (at 136.8044 116.332) (size 0.8) (drill 0.4) (layers F.Cu B.Cu) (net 20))
 (segment (start 133.698 114.808) (end 135.2804 114.808) (width 0.25) (layer F.Cu) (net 20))
 (segment (start 135.2804 114.808) (end 136.8044 116.332) (width 0.25) (layer F.Cu) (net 20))
 (segment (start 136.8044 120.4976) (end 136.652 120.65) (width 0.25) (layer B.Cu) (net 20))
 (segment (start 136.8044 116.332) (end 136.8044 120.4976) (width 0.25) (layer B.Cu) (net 20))
 (segment (start 150.622 122.428) (end 143.764 115.57) (width 0.25) (layer F.Cu) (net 16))
 (segment (start 150.622 124.968) (end 150.622 122.428) (width 0.25) (layer F.Cu) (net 16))
 (segment (start 142.992653 114.798653) (end 143.764 115.57) (width 0.25) (layer F.Cu) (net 16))
 (segment (start 141.106999 112.912999) (end 142.992653 114.798653) (width 0.25) (layer F.Cu) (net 16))
 (segment (start 138.107997 112.912999) (end 141.106999 112.912999) (width 0.25) (layer F.Cu) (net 16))
 (segment (start 138.022999 112.828001) (end 138.107997 112.912999) (width 0.25) (layer F.Cu) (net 16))
 (segment (start 138.022999 108.533001) (end 138.022999 112.828001) (width 0.25) (layer F.Cu) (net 16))
 (segment (start 138.098 108.458) (end 138.022999 108.533001) (width 0.25) (layer F.Cu) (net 16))
 (segment (start 139.098 108.458) (end 138.098 108.458) (width 0.25) (layer F.Cu) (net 16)))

